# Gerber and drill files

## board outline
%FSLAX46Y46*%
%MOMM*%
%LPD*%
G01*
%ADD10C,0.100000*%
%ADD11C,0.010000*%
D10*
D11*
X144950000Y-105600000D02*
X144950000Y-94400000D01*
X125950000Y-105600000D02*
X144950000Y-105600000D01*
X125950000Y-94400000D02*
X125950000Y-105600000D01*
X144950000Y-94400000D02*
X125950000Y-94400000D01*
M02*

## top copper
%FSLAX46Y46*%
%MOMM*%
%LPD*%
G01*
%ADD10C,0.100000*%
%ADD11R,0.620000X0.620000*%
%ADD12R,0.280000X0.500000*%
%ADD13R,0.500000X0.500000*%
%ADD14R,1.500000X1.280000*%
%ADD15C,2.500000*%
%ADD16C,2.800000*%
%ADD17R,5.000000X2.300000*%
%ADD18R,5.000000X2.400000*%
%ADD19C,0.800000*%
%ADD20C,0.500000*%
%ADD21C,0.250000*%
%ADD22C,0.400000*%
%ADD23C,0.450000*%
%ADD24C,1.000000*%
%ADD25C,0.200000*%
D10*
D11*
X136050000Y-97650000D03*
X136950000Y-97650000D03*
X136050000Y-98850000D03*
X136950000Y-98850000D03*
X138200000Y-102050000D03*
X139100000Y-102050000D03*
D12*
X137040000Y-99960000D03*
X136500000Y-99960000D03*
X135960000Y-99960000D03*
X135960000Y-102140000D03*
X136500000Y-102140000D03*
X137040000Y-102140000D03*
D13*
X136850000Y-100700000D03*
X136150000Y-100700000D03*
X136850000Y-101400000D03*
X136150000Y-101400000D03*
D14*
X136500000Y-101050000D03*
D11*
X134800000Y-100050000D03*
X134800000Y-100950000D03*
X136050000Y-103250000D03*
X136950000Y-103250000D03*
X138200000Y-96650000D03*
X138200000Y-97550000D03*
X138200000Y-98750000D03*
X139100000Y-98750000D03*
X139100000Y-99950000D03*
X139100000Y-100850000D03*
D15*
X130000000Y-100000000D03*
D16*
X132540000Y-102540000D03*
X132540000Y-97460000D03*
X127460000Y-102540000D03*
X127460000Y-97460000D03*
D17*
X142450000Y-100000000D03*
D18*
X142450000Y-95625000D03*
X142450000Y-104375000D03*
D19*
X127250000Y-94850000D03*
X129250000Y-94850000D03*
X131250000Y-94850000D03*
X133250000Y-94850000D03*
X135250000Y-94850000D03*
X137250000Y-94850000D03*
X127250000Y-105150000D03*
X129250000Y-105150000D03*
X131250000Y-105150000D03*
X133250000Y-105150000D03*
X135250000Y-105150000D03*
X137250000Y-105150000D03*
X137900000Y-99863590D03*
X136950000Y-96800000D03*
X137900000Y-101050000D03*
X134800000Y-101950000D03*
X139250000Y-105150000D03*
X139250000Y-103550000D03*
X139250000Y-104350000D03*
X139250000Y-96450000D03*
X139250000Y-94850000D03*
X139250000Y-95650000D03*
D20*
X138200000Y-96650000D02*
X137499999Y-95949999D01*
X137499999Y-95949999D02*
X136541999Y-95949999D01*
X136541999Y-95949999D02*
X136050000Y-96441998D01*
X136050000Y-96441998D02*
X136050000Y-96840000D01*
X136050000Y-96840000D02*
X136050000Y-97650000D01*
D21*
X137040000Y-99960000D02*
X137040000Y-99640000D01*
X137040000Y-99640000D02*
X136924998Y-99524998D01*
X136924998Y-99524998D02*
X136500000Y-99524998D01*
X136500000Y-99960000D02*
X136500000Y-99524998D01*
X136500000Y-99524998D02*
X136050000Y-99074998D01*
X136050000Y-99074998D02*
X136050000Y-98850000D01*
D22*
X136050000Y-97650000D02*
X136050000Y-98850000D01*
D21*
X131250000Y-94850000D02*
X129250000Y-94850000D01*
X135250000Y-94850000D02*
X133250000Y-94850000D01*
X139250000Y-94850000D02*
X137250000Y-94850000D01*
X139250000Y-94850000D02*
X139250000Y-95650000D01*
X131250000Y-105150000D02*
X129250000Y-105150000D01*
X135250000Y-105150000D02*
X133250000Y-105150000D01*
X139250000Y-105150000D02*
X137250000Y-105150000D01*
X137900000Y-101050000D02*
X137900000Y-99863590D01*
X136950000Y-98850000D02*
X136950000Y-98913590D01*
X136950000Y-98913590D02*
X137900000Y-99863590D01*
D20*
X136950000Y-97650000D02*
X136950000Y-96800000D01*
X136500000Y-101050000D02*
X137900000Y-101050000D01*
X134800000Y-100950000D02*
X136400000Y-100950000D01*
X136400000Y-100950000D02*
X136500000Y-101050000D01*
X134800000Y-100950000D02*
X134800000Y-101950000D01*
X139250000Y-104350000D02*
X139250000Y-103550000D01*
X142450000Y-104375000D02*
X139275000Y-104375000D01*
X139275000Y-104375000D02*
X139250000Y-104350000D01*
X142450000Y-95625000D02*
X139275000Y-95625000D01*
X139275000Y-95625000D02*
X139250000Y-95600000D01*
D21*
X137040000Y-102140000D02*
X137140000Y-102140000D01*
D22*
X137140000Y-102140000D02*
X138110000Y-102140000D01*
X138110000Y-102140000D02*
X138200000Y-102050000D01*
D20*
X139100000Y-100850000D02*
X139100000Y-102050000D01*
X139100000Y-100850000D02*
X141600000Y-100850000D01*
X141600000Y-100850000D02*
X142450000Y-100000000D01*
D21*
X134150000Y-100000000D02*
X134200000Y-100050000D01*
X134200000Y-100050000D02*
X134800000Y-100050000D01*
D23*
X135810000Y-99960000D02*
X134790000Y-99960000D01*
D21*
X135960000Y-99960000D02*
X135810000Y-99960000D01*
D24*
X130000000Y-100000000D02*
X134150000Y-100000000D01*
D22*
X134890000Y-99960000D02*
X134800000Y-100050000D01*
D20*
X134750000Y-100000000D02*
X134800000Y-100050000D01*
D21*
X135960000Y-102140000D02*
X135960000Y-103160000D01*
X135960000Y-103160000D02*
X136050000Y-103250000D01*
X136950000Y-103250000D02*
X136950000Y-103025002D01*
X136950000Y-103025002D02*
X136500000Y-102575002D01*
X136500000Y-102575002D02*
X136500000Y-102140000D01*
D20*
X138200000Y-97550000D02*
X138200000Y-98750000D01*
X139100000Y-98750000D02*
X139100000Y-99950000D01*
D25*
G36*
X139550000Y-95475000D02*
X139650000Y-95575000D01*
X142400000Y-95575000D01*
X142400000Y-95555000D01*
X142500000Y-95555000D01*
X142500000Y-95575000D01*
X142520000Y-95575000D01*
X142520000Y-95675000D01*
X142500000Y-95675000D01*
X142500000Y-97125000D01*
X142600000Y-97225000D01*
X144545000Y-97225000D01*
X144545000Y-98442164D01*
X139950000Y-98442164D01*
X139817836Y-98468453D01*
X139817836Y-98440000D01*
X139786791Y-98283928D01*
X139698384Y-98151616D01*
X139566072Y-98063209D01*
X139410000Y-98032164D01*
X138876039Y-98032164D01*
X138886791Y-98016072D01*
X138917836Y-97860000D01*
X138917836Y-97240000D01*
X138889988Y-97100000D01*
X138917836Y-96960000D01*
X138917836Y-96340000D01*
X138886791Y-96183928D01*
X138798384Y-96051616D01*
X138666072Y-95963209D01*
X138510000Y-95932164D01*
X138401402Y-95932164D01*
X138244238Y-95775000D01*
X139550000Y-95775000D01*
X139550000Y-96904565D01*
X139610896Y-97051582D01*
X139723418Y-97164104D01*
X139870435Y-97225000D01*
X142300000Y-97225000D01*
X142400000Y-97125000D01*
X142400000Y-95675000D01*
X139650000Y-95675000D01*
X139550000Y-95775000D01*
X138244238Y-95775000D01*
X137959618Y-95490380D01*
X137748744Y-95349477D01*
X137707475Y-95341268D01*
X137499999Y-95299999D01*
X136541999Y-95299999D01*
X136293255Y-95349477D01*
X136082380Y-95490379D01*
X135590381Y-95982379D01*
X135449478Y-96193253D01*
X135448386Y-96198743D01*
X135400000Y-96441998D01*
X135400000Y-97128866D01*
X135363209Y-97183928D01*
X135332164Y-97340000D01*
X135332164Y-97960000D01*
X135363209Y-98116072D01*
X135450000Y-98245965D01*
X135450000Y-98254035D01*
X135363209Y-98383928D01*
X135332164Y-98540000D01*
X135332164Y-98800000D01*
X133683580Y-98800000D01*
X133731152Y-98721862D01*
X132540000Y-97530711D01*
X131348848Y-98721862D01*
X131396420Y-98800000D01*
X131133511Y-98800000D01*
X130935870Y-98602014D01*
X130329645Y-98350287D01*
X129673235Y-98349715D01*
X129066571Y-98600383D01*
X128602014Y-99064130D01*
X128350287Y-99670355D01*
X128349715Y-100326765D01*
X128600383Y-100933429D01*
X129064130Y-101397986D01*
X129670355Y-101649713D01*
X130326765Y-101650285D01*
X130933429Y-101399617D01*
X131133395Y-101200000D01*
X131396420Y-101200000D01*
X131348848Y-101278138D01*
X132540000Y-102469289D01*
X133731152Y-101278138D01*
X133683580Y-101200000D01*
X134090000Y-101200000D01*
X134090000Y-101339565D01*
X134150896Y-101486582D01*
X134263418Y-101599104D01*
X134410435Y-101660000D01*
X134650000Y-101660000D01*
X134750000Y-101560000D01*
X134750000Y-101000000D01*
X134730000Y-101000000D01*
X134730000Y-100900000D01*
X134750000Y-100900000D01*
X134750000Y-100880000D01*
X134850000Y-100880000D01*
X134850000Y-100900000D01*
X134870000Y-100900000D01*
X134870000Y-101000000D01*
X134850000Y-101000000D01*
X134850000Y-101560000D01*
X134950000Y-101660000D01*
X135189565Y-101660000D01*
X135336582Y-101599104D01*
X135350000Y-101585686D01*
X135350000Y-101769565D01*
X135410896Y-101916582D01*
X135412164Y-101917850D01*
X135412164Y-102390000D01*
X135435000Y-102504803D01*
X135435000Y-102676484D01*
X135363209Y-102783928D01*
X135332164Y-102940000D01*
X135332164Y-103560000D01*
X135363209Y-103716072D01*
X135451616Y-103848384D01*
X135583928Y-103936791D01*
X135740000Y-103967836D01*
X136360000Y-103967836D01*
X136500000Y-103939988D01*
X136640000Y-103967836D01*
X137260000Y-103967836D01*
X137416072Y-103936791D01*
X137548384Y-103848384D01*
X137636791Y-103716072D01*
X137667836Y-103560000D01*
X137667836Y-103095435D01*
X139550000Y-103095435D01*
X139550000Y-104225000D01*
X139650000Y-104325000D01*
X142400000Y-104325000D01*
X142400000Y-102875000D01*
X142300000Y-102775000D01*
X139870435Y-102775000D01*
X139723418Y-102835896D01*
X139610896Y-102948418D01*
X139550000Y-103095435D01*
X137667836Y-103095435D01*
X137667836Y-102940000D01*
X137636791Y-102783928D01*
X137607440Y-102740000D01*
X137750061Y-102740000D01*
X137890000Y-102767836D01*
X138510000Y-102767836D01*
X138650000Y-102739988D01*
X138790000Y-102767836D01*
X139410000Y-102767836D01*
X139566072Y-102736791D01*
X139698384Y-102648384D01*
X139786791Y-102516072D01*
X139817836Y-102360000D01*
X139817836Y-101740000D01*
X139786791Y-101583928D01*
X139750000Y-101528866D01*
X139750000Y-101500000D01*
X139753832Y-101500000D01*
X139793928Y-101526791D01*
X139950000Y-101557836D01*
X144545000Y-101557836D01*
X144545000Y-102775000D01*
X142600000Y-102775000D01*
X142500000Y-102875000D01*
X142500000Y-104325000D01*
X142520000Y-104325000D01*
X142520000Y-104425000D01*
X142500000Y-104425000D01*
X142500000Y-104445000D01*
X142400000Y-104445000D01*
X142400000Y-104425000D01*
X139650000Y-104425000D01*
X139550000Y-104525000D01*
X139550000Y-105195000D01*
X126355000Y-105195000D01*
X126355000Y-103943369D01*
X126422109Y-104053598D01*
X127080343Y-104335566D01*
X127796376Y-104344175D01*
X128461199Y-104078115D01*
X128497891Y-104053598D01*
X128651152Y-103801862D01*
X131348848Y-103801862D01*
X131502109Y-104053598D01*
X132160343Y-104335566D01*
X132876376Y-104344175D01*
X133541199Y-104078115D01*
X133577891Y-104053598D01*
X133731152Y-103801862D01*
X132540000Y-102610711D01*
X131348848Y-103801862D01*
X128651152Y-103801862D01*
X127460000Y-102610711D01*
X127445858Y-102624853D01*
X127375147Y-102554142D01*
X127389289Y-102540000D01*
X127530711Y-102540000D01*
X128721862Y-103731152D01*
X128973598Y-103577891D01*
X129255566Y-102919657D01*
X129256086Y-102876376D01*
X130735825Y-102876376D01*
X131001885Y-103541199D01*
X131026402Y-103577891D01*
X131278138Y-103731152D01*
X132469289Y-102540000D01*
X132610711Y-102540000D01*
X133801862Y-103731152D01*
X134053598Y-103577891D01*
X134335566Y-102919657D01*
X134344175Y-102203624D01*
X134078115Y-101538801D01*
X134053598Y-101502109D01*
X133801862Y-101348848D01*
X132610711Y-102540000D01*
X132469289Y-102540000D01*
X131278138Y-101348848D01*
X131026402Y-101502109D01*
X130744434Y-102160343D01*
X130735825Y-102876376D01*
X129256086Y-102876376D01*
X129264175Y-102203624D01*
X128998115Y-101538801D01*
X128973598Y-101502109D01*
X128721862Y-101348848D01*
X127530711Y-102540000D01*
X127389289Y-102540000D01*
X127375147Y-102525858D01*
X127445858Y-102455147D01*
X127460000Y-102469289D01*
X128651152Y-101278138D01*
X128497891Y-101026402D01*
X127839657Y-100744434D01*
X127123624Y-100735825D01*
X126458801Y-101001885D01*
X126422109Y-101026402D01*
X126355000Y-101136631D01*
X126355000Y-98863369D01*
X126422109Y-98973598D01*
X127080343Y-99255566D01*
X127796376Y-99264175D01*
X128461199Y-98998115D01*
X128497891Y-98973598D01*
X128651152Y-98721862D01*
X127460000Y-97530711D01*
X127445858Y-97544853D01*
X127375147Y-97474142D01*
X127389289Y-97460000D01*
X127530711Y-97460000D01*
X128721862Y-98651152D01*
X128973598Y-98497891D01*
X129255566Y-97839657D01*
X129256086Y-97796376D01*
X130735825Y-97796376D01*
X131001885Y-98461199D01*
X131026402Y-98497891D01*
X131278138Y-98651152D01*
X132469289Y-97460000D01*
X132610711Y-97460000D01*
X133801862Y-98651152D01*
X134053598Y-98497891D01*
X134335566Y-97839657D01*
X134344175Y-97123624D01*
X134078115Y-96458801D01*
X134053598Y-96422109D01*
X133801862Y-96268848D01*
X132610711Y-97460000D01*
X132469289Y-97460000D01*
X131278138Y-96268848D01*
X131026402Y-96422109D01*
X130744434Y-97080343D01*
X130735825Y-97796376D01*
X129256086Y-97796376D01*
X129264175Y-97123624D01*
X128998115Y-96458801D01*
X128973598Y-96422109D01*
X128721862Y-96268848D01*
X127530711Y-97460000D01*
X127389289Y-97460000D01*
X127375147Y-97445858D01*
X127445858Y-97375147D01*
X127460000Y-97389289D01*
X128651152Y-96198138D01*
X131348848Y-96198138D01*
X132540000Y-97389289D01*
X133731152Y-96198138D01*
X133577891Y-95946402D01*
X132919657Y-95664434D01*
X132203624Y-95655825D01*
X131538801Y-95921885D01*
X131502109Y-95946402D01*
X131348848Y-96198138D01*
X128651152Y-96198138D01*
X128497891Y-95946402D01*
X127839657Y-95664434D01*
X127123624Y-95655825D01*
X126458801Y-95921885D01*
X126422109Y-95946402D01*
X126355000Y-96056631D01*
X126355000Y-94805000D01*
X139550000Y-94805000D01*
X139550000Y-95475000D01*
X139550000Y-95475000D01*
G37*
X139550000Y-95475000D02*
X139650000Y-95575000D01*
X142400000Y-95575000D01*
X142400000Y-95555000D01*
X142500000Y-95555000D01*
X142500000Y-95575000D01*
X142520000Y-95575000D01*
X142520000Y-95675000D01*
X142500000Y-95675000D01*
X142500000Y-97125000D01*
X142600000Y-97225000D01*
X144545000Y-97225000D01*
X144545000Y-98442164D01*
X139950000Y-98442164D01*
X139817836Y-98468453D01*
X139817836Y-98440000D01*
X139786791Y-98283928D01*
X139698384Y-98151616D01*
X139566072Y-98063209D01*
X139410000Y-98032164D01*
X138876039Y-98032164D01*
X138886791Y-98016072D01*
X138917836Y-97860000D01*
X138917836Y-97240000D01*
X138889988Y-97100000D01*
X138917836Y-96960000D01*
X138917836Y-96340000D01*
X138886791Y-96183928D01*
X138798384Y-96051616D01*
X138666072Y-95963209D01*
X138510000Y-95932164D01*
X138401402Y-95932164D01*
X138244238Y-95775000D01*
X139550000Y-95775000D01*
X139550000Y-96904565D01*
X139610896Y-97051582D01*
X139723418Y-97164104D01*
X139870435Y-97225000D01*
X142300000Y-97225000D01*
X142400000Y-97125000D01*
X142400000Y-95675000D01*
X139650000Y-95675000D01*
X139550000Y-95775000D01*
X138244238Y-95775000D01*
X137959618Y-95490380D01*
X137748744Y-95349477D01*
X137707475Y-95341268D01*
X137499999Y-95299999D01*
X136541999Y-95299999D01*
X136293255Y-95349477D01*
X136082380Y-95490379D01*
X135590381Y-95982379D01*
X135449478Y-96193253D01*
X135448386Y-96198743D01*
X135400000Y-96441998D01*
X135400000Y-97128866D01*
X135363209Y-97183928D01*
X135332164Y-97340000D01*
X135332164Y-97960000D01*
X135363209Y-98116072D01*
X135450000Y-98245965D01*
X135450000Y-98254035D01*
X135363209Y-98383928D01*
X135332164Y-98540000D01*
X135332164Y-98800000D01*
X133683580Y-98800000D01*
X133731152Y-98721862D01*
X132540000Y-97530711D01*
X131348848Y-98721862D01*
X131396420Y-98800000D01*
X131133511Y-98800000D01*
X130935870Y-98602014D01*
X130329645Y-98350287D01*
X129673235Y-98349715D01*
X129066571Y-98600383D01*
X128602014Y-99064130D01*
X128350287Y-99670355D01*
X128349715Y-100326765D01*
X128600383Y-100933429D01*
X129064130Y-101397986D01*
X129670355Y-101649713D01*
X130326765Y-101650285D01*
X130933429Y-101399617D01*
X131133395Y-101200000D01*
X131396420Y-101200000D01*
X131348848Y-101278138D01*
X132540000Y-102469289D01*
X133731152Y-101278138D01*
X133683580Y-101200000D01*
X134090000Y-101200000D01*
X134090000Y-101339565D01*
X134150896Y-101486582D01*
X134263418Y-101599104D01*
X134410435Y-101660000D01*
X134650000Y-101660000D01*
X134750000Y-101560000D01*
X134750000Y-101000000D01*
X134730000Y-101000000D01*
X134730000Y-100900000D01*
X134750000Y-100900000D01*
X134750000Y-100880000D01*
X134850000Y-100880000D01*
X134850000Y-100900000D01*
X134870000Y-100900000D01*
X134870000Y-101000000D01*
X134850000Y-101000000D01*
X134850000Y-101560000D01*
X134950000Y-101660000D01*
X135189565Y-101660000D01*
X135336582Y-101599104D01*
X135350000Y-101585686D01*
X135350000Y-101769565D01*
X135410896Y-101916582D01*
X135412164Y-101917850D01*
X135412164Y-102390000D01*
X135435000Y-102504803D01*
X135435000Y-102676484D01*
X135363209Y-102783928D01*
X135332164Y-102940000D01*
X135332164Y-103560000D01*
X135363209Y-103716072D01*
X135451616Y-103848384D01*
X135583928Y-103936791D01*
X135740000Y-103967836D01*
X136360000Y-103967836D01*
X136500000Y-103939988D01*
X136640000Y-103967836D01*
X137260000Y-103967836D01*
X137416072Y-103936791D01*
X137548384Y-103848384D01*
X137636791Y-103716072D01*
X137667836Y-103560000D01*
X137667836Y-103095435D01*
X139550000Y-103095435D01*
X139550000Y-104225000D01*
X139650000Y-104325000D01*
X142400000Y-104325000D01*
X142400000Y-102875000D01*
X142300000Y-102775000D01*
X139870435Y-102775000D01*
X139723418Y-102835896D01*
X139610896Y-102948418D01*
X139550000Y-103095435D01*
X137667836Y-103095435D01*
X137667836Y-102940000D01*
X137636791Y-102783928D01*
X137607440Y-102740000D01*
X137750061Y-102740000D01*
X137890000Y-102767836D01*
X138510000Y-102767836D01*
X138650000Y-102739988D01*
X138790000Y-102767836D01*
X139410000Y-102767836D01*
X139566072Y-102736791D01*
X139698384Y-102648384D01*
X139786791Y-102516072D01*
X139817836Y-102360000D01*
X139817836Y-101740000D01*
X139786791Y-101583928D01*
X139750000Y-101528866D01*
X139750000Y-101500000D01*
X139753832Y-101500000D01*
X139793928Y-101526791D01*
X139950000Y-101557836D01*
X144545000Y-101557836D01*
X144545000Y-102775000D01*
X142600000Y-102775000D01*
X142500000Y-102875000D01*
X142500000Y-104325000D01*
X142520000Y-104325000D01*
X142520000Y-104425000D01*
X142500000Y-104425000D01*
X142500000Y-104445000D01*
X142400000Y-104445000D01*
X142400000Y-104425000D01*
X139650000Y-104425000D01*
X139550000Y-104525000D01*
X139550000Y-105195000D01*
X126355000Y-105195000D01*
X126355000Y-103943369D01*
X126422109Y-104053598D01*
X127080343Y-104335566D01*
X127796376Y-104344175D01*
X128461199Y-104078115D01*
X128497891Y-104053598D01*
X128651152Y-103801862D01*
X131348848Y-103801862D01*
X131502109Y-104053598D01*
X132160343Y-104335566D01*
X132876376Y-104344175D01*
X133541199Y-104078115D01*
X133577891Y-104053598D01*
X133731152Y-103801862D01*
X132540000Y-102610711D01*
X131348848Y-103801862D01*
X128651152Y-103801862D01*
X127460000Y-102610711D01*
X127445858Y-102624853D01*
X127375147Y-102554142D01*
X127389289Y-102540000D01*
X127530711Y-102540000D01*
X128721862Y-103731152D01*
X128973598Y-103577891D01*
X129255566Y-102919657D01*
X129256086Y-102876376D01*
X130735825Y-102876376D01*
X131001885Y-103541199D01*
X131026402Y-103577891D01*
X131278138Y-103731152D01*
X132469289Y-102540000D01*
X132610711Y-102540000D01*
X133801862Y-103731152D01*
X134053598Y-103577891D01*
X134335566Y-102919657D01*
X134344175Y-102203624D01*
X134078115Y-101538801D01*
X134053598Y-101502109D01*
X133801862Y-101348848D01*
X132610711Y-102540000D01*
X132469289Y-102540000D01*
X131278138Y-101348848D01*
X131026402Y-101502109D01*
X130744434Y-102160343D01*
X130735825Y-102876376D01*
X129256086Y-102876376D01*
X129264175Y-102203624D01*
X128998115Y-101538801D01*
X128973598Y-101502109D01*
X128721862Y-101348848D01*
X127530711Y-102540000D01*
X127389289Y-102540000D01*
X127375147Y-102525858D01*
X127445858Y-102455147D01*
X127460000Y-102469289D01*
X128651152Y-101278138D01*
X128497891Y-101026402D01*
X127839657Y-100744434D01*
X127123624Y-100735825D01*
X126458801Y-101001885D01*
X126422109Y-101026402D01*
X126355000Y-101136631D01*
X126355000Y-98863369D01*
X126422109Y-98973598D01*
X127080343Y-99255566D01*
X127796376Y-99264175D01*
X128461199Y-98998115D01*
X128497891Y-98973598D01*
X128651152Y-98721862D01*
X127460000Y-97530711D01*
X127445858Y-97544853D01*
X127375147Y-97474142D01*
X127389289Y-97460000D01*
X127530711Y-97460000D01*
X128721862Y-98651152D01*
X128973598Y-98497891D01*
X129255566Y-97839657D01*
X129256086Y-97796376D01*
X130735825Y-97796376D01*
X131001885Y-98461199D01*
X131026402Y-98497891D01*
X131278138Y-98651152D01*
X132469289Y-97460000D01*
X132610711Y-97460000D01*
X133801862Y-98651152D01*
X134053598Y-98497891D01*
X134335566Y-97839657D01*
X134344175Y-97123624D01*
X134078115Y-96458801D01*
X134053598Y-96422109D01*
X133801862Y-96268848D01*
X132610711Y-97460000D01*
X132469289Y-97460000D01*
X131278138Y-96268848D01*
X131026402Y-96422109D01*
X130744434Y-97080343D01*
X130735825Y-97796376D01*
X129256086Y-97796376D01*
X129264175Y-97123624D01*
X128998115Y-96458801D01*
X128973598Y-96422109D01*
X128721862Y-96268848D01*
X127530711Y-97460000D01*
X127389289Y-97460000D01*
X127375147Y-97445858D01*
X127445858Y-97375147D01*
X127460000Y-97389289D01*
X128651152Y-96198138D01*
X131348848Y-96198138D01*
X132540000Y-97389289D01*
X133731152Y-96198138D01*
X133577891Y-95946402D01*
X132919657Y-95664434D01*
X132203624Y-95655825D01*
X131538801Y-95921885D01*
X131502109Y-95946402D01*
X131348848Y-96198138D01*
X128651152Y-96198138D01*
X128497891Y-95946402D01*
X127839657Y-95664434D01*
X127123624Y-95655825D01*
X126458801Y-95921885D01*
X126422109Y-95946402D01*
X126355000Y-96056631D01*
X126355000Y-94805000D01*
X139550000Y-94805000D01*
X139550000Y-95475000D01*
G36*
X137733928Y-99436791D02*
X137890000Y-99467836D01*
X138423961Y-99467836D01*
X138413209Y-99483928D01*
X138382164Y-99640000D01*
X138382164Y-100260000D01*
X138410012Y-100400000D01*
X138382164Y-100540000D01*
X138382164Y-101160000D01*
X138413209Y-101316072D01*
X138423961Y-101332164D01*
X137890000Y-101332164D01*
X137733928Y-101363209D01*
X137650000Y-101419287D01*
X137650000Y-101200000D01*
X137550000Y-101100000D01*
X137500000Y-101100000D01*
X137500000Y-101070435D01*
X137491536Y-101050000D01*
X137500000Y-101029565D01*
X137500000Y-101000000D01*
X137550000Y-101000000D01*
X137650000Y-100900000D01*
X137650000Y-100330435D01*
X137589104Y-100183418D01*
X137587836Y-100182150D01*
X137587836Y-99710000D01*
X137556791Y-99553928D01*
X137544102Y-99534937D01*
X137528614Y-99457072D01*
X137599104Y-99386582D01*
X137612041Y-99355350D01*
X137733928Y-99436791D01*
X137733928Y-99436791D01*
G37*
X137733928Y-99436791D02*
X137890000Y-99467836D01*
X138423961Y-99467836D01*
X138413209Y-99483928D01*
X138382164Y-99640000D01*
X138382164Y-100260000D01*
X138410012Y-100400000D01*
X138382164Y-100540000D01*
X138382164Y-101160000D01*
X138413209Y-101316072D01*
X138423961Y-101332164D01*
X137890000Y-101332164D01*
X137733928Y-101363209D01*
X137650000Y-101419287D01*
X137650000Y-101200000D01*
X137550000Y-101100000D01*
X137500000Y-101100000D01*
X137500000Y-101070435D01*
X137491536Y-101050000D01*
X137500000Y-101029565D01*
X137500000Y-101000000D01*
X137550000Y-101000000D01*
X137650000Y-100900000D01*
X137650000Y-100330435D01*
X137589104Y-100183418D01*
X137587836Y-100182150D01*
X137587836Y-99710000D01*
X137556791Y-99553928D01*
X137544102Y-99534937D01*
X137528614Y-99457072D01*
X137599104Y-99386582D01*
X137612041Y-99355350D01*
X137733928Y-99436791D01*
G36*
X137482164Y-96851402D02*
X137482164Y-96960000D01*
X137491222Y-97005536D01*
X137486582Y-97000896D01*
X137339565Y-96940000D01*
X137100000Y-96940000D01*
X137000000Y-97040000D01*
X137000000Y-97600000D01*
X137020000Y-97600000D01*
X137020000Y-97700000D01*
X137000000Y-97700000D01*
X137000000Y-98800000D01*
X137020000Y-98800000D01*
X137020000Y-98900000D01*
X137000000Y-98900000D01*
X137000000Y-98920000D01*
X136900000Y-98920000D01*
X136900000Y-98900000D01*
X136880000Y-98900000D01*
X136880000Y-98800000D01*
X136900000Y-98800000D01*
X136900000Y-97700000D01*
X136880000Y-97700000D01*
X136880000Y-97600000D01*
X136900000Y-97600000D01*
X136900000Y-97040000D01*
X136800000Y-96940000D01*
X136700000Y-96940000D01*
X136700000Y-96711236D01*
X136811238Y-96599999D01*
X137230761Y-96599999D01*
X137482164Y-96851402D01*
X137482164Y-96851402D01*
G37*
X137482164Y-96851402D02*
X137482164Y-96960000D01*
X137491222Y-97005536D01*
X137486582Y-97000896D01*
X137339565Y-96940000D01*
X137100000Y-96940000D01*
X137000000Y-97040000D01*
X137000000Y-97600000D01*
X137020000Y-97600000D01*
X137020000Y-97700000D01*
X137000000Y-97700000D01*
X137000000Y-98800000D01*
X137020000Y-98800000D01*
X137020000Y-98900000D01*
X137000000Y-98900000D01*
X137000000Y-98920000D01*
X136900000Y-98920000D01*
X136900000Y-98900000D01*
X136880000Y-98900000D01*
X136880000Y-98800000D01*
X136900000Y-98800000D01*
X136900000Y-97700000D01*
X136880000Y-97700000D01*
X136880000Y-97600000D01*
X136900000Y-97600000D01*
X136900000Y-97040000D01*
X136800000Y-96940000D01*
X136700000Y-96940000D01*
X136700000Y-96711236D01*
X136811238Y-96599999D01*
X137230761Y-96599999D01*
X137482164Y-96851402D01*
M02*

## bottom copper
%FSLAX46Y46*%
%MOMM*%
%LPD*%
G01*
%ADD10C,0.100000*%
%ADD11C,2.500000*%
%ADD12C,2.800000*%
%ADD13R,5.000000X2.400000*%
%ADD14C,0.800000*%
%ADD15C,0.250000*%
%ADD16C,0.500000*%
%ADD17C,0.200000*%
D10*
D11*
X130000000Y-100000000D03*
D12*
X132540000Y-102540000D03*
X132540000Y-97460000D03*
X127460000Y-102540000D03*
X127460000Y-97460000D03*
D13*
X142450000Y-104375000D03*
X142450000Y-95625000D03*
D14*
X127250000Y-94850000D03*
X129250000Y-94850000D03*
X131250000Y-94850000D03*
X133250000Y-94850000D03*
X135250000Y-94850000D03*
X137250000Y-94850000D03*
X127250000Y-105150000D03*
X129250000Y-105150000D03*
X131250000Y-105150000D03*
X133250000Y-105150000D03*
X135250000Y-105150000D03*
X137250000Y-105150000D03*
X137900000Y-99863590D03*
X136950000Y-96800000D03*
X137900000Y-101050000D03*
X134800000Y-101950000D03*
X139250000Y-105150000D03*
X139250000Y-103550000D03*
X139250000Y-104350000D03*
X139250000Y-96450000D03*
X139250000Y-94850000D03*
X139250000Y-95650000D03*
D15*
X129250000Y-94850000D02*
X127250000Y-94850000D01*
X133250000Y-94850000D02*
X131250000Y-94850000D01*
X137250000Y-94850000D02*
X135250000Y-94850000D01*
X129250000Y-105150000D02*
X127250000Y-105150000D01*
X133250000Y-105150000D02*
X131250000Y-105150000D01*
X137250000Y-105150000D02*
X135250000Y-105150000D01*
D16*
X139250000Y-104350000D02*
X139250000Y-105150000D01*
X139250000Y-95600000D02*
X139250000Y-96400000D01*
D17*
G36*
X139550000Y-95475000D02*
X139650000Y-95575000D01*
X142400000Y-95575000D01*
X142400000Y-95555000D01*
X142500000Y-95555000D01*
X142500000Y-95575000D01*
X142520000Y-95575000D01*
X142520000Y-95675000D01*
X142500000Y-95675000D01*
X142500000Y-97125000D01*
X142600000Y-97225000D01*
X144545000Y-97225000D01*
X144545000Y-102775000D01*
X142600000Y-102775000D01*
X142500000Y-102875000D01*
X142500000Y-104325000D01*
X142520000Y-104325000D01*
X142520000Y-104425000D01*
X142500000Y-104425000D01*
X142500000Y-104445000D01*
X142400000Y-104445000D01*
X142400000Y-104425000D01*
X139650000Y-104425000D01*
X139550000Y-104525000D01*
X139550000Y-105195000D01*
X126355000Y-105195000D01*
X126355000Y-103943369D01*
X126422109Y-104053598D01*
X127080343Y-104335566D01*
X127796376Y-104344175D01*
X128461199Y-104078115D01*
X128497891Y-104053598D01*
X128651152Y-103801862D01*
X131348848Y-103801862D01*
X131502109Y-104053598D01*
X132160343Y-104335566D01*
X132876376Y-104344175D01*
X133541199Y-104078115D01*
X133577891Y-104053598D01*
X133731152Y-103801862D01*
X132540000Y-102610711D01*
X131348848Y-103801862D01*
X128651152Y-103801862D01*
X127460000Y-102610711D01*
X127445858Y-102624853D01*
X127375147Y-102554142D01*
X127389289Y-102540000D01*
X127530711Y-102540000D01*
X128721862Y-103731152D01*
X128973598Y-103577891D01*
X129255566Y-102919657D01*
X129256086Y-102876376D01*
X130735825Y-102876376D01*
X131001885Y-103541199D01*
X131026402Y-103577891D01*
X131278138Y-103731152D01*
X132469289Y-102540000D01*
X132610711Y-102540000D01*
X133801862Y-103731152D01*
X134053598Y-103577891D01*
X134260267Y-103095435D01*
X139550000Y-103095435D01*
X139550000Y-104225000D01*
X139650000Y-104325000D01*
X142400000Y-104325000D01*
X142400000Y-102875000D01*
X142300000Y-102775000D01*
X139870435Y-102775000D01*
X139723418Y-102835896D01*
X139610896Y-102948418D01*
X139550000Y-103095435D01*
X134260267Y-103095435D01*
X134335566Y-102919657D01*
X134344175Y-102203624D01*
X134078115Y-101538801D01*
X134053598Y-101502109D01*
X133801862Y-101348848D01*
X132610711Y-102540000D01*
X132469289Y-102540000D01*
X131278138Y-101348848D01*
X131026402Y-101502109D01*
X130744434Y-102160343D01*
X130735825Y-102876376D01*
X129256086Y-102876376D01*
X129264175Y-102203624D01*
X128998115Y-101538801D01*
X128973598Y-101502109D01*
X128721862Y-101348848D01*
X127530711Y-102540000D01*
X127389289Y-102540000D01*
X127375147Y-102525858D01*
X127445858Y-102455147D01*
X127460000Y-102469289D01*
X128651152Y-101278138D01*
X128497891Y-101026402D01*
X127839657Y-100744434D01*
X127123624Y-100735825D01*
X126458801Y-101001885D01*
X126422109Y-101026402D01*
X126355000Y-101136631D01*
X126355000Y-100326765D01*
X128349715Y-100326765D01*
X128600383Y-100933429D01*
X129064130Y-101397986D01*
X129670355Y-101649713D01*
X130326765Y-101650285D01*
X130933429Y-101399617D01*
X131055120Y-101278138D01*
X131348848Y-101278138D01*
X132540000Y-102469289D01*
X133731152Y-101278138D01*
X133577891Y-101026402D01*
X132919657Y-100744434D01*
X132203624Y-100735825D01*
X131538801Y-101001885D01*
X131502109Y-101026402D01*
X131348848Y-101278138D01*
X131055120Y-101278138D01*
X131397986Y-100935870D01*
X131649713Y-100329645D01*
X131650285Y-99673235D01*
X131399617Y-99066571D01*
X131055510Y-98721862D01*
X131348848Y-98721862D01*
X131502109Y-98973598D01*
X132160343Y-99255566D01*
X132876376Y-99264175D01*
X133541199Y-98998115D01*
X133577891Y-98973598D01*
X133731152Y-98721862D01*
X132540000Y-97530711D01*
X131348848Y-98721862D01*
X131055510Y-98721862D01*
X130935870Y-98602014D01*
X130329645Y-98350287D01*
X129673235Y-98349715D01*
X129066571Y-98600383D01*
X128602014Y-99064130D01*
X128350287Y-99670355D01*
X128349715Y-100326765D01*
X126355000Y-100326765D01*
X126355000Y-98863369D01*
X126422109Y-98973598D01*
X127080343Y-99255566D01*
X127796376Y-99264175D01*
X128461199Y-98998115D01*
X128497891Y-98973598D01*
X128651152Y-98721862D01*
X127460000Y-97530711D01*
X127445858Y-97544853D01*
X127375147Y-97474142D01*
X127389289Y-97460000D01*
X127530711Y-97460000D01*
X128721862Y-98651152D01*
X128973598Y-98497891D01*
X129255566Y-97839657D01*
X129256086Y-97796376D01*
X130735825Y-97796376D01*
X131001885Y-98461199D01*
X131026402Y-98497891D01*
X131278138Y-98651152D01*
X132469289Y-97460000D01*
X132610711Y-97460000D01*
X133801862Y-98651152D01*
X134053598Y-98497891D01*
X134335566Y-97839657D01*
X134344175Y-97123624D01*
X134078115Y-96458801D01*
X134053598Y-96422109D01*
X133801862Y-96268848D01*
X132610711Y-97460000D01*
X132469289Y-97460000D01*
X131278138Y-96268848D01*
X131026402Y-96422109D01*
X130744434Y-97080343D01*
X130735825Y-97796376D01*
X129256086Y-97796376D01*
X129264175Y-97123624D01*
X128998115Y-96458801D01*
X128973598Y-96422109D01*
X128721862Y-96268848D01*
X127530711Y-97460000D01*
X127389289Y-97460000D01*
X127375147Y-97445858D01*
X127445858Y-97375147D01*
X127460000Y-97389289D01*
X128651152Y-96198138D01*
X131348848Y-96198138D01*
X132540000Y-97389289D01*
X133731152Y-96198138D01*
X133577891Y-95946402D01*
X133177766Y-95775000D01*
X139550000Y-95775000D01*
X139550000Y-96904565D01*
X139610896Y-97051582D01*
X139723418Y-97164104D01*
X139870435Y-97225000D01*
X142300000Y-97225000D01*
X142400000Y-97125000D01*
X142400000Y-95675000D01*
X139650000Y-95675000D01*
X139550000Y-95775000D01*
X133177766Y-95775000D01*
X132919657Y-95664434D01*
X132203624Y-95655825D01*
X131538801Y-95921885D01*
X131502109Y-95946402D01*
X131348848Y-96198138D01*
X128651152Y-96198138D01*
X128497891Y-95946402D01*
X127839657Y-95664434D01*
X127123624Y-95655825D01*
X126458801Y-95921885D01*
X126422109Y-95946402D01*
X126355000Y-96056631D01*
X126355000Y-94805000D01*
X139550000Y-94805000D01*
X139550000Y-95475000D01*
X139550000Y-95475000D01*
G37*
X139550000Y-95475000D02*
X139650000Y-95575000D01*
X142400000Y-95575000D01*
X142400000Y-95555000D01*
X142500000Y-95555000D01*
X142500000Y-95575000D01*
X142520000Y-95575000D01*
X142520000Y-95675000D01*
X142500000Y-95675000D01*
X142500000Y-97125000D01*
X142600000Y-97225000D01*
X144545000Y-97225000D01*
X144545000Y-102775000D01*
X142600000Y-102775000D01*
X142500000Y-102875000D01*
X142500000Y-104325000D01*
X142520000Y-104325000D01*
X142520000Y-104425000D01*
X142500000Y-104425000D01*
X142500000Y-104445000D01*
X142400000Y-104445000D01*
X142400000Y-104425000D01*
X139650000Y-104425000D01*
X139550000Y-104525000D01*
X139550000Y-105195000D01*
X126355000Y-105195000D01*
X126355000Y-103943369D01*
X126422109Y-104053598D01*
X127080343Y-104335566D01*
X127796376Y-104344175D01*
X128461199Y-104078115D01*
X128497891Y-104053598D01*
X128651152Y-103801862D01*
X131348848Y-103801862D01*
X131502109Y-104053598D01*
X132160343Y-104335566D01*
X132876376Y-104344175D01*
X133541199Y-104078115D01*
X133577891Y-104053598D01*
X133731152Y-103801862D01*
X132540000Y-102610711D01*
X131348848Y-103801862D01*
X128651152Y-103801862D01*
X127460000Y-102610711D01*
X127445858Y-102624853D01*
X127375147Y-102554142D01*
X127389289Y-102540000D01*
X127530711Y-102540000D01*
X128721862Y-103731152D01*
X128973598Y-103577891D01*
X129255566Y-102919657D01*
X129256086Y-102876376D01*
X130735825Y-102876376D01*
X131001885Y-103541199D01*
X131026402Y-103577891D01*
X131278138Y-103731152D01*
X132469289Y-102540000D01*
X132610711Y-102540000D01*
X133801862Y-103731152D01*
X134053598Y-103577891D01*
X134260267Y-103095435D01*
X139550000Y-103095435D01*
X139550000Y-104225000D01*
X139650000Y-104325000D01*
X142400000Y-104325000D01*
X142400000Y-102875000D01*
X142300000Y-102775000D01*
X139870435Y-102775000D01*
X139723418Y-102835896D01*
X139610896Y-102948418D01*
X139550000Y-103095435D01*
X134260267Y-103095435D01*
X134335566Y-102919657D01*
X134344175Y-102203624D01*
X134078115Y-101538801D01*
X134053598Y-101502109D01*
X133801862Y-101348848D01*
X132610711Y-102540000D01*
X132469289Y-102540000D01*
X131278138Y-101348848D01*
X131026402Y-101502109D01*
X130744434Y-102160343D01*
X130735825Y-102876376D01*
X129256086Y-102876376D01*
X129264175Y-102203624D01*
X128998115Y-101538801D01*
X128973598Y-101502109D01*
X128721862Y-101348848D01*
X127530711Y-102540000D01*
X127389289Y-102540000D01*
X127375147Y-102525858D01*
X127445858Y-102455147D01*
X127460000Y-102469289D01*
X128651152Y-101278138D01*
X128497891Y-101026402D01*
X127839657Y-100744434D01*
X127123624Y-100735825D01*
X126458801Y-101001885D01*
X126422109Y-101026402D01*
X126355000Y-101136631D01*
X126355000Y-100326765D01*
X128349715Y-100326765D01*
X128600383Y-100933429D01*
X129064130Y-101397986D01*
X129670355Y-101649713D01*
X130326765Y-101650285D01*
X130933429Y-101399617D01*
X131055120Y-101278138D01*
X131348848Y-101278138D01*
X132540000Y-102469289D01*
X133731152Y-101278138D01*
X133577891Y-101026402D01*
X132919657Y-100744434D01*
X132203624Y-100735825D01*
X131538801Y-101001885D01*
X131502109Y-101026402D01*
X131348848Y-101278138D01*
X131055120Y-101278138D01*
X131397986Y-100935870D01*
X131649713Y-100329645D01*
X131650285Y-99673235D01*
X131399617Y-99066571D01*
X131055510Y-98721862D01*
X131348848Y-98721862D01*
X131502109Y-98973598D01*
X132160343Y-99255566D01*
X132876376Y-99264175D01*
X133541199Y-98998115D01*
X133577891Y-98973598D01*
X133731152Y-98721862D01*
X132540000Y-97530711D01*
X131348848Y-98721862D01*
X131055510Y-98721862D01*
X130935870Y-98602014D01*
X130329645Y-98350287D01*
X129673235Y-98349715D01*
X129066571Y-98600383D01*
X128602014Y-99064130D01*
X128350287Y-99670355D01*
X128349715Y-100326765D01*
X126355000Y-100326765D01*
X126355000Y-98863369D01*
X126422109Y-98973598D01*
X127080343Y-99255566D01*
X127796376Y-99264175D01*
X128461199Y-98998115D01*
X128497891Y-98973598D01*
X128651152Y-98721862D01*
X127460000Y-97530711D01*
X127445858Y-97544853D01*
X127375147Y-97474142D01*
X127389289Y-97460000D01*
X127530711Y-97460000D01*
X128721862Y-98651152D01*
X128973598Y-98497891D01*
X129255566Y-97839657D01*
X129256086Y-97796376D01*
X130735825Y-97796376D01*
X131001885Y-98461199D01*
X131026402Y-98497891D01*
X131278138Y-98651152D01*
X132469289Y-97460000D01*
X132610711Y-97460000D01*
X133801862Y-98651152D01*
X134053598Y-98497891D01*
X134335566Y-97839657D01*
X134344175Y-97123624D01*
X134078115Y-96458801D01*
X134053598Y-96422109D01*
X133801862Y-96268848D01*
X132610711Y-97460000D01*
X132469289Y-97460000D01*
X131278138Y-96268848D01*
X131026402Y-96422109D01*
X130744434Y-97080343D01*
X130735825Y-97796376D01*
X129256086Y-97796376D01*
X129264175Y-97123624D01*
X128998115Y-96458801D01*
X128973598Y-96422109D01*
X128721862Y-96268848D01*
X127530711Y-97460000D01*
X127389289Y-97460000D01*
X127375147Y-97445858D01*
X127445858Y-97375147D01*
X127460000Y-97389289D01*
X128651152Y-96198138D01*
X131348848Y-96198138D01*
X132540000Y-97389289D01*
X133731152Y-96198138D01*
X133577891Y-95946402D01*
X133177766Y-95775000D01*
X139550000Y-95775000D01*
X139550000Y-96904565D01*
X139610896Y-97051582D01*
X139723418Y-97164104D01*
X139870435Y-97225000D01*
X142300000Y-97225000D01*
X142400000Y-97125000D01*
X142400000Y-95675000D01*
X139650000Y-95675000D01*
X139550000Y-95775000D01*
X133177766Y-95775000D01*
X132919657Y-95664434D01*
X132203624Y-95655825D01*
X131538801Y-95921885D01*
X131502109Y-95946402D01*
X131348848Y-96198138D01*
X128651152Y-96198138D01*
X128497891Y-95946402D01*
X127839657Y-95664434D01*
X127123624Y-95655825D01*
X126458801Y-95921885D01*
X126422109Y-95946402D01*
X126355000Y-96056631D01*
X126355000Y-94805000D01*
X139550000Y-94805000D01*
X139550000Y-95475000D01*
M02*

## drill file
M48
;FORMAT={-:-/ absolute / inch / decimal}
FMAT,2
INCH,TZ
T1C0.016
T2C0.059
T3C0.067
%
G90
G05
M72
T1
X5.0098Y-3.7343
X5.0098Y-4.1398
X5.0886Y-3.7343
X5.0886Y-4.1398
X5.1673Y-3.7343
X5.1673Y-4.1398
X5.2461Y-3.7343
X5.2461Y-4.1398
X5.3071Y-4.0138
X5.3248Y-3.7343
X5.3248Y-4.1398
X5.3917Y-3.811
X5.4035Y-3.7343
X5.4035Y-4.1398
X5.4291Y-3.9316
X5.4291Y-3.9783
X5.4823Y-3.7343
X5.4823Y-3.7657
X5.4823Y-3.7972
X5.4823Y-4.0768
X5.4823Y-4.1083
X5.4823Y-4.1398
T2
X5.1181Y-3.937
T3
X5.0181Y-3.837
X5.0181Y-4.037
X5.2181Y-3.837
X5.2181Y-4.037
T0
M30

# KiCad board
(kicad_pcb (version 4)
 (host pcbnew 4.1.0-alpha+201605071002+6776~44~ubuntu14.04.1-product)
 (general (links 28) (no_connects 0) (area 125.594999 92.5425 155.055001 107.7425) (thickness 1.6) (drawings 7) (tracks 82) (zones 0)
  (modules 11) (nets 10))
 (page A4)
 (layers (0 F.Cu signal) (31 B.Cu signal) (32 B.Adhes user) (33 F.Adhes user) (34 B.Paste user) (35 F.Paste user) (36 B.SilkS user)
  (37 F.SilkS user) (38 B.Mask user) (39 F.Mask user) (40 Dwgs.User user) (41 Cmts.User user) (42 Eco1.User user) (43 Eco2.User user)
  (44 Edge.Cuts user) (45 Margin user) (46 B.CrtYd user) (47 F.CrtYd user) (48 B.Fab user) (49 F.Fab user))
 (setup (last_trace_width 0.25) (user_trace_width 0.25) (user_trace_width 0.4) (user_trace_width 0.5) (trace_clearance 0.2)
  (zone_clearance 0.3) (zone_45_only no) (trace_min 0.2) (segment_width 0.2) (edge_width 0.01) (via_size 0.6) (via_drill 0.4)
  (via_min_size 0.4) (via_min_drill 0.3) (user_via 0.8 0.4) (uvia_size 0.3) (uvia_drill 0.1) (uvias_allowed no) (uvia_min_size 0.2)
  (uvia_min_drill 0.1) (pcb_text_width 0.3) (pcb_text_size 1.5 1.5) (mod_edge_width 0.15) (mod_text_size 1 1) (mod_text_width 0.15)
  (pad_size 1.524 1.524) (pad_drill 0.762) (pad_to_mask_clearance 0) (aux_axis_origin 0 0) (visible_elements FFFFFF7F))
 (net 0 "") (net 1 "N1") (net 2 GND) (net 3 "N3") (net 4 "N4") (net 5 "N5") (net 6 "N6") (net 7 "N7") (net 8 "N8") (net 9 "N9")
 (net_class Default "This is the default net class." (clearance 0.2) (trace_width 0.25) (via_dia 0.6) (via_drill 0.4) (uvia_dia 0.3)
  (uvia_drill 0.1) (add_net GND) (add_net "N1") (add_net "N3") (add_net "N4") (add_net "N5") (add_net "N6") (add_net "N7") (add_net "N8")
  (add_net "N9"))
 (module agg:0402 (layer F.Cu) (at 136.5 97.65)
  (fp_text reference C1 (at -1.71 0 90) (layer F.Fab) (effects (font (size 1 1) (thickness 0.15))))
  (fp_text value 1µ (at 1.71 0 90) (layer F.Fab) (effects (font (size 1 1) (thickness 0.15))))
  (pad 1 smd rect (at -0.45 0) (size 0.62 0.62) (layers F.Cu F.Paste F.Mask) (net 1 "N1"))
  (pad 2 smd rect (at 0.45 0) (size 0.62 0.62) (layers F.Cu F.Paste F.Mask) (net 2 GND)))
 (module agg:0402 (layer F.Cu) (at 136.5 98.85)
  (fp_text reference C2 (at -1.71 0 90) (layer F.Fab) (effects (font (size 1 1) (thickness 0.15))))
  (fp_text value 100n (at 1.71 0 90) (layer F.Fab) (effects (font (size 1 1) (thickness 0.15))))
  (pad 1 smd rect (at -0.45 0) (size 0.62 0.62) (layers F.Cu F.Paste F.Mask) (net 1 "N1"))
  (pad 2 smd rect (at 0.45 0) (size 0.62 0.62) (layers F.Cu F.Paste F.Mask) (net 2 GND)))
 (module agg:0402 (layer F.Cu) (at 138.65 102.05)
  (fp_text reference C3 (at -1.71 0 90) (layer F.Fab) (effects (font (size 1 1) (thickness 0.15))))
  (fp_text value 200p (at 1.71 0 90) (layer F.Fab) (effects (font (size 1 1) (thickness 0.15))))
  (pad 1 smd rect (at -0.45 0) (size 0.62 0.62) (layers F.Cu F.Paste F.Mask) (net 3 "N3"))
  (pad 2 smd rect (at 0.45 0) (size 0.62 0.62) (layers F.Cu F.Paste F.Mask) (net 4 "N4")))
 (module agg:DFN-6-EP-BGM (layer F.Cu) (at 136.5 101.05 270)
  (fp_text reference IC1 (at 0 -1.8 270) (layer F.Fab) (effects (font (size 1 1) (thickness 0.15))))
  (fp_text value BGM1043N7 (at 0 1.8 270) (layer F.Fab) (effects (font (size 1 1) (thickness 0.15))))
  (pad 1 smd rect (at -1.09 -0.54 270) (size 0.5 0.28) (layers F.Cu F.Paste F.Mask) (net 1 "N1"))
  (pad 2 smd rect (at -1.09 0 270) (size 0.5 0.28) (layers F.Cu F.Paste F.Mask) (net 1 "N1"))
  (pad 3 smd rect (at -1.09 0.54 270) (size 0.5 0.28) (layers F.Cu F.Paste F.Mask) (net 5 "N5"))
  (pad 4 smd rect (at 1.09 0.54 270) (size 0.5 0.28) (layers F.Cu F.Paste F.Mask) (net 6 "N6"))
  (pad 5 smd rect (at 1.09 0 270) (size 0.5 0.28) (layers F.Cu F.Paste F.Mask) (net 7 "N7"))
  (pad 6 smd rect (at 1.09 -0.54 270) (size 0.5 0.28) (layers F.Cu F.Paste F.Mask) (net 3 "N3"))
  (pad EP smd rect (at -0.35 -0.35 270) (size 0.5 0.5) (layers F.Cu F.Paste) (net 2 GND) (solder_paste_margin 0.001))
  (pad EP smd rect (at -0.35 0.35 270) (size 0.5 0.5) (layers F.Cu F.Paste) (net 2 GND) (solder_paste_margin 0.001))
  (pad EP smd rect (at 0.35 -0.35 270) (size 0.5 0.5) (layers F.Cu F.Paste) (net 2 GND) (solder_paste_margin 0.001))
  (pad EP smd rect (at 0.35 0.35 270) (size 0.5 0.5) (layers F.Cu F.Paste) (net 2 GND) (solder_paste_margin 0.001))
  (pad EP smd rect (at 0 0 270) (size 1.28 1.5) (layers F.Cu F.Mask) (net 2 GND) (solder_mask_margin 0.001)))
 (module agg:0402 (layer F.Cu) (at 134.8 100.5 270)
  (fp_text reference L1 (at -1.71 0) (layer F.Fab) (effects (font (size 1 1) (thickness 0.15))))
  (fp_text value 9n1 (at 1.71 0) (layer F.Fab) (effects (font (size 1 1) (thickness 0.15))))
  (pad 1 smd rect (at -0.45 0 270) (size 0.62 0.62) (layers F.Cu F.Paste F.Mask) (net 5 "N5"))
  (pad 2 smd rect (at 0.45 0 270) (size 0.62 0.62) (layers F.Cu F.Paste F.Mask) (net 2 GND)))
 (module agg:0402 (layer F.Cu) (at 136.5 103.25)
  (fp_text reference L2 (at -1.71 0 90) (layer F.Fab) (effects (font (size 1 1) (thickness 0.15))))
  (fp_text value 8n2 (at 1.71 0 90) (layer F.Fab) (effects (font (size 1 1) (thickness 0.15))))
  (pad 1 smd rect (at -0.45 0) (size 0.62 0.62) (layers F.Cu F.Paste F.Mask) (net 6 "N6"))
  (pad 2 smd rect (at 0.45 0) (size 0.62 0.62) (layers F.Cu F.Paste F.Mask) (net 7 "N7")))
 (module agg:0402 (layer F.Cu) (at 138.2 97.1 270)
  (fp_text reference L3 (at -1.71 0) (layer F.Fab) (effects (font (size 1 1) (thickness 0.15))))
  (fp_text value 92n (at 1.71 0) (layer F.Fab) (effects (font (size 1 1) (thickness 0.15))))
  (pad 1 smd rect (at -0.45 0 270) (size 0.62 0.62) (layers F.Cu F.Paste F.Mask) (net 1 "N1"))
  (pad 2 smd rect (at 0.45 0 270) (size 0.62 0.62) (layers F.Cu F.Paste F.Mask) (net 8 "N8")))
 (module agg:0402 (layer F.Cu) (at 138.65 98.75)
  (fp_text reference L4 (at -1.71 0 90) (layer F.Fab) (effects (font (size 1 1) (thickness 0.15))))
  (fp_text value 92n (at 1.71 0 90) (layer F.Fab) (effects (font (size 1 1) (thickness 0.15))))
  (pad 1 smd rect (at -0.45 0) (size 0.62 0.62) (layers F.Cu F.Paste F.Mask) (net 8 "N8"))
  (pad 2 smd rect (at 0.45 0) (size 0.62 0.62) (layers F.Cu F.Paste F.Mask) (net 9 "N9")))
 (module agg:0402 (layer F.Cu) (at 139.1 100.4 270)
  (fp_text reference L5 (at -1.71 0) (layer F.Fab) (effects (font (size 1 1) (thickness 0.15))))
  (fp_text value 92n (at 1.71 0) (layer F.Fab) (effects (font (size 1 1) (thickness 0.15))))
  (pad 1 smd rect (at -0.45 0 270) (size 0.62 0.62) (layers F.Cu F.Paste F.Mask) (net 9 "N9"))
  (pad 2 smd rect (at 0.45 0 270) (size 0.62 0.62) (layers F.Cu F.Paste F.Mask) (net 4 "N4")))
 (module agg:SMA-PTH (layer F.Cu) (at 130 100)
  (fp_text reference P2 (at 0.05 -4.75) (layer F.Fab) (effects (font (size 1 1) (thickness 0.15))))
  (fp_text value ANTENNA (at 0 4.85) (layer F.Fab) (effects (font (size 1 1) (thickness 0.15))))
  (pad 1 thru_hole circle (at 0 0) (size 2.5 2.5) (drill 1.5) (layers *.Cu *.Mask F.SilkS) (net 5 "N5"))
  (pad 2 thru_hole circle (at 2.54 2.54) (size 2.8 2.8) (drill 1.7) (layers *.Cu *.Mask F.SilkS) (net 2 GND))
  (pad 2 thru_hole circle (at 2.54 -2.54) (size 2.8 2.8) (drill 1.7) (layers *.Cu *.Mask F.SilkS) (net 2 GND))
  (pad 2 thru_hole circle (at -2.54 2.54) (size 2.8 2.8) (drill 1.7) (layers *.Cu *.Mask F.SilkS) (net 2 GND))
  (pad 2 thru_hole circle (at -2.54 -2.54) (size 2.8 2.8) (drill 1.7) (layers *.Cu *.Mask F.SilkS) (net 2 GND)))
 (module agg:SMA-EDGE (layer F.Cu) (at 142.45 100 270)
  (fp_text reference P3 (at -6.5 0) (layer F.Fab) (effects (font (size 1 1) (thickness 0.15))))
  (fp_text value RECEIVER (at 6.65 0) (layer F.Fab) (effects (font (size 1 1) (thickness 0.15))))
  (pad 1 smd rect (at 0 0 270) (size 2.3 5) (layers F.Cu F.Paste F.Mask) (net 4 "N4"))
  (pad 2 smd rect (at 4.375 0 270) (size 2.4 5) (layers B.Cu B.Paste B.Mask) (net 2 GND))
  (pad 2 smd rect (at -4.375 0 270) (size 2.4 5) (layers B.Cu B.Paste B.Mask) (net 2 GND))
  (pad 2 smd rect (at -4.375 0 270) (size 2.4 5) (layers F.Cu F.Paste F.Mask) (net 2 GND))
  (pad 2 smd rect (at 4.375 0 270) (size 2.4 5) (layers F.Cu F.Paste F.Mask) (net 2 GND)))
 (gr_line (start 144.95 105.6) (end 144.95 94.4) (layer Edge.Cuts) (width 0.01))
 (gr_line (start 125.95 105.6) (end 144.95 105.6) (layer Edge.Cuts) (width 0.01))
 (gr_line (start 125.95 94.4) (end 125.95 105.6) (layer Edge.Cuts) (width 0.01))
 (gr_line (start 144.95 94.4) (end 125.95 94.4) (layer Edge.Cuts) (width 0.01))
 (segment (start 138.2 96.65) (end 137.499999 95.949999) (width 0.5) (layer F.Cu) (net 1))
 (segment (start 137.499999 95.949999) (end 136.541999 95.949999) (width 0.5) (layer F.Cu) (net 1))
 (segment (start 136.541999 95.949999) (end 136.05 96.441998) (width 0.5) (layer F.Cu) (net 1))
 (segment (start 136.05 96.441998) (end 136.05 96.84) (width 0.5) (layer F.Cu) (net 1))
 (segment (start 136.05 96.84) (end 136.05 97.65) (width 0.5) (layer F.Cu) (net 1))
 (segment (start 137.04 99.96) (end 137.04 99.64) (width 0.25) (layer F.Cu) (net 1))
 (segment (start 137.04 99.64) (end 136.924998 99.524998) (width 0.25) (layer F.Cu) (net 1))
 (segment (start 136.924998 99.524998) (end 136.5 99.524998) (width 0.25) (layer F.Cu) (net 1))
 (segment (start 136.5 99.96) (end 136.5 99.524998) (width 0.25) (layer F.Cu) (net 1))
 (segment (start 136.5 99.524998) (end 136.05 99.074998) (width 0.25) (layer F.Cu) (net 1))
 (segment (start 136.05 99.074998) (end 136.05 98.85) (width 0.25) (layer F.Cu) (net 1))
 (segment (start 136.05 97.65) (end 136.05 98.85) (width 0.4) (layer F.Cu) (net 1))
 (segment (start 129.25 94.85) (end 127.25 94.85) (width 0.25) (layer B.Cu) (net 2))
 (via (at 127.25 94.85) (size 0.8) (drill 0.4) (layers F.Cu B.Cu) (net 2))
 (segment (start 131.25 94.85) (end 129.25 94.85) (width 0.25) (layer F.Cu) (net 2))
 (via (at 129.25 94.85) (size 0.8) (drill 0.4) (layers F.Cu B.Cu) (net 2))
 (segment (start 133.25 94.85) (end 131.25 94.85) (width 0.25) (layer B.Cu) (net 2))
 (via (at 131.25 94.85) (size 0.8) (drill 0.4) (layers F.Cu B.Cu) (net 2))
 (segment (start 135.25 94.85) (end 133.25 94.85) (width 0.25) (layer F.Cu) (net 2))
 (via (at 133.25 94.85) (size 0.8) (drill 0.4) (layers F.Cu B.Cu) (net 2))
 (segment (start 137.25 94.85) (end 135.25 94.85) (width 0.25) (layer B.Cu) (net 2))
 (via (at 135.25 94.85) (size 0.8) (drill 0.4) (layers F.Cu B.Cu) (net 2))
 (segment (start 139.25 94.85) (end 137.25 94.85) (width 0.25) (layer F.Cu) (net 2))
 (via (at 137.25 94.85) (size 0.8) (drill 0.4) (layers F.Cu B.Cu) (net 2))
 (segment (start 139.25 94.85) (end 139.25 95.65) (width 0.25) (layer F.Cu) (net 2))
 (segment (start 129.25 105.15) (end 127.25 105.15) (width 0.25) (layer B.Cu) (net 2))
 (via (at 127.25 105.15) (size 0.8) (drill 0.4) (layers F.Cu B.Cu) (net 2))
 (segment (start 131.25 105.15) (end 129.25 105.15) (width 0.25) (layer F.Cu) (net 2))
 (via (at 129.25 105.15) (size 0.8) (drill 0.4) (layers F.Cu B.Cu) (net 2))
 (segment (start 133.25 105.15) (end 131.25 105.15) (width 0.25) (layer B.Cu) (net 2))
 (via (at 131.25 105.15) (size 0.8) (drill 0.4) (layers F.Cu B.Cu) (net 2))
 (segment (start 135.25 105.15) (end 133.25 105.15) (width 0.25) (layer F.Cu) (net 2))
 (via (at 133.25 105.15) (size 0.8) (drill 0.4) (layers F.Cu B.Cu) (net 2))
 (segment (start 137.25 105.15) (end 135.25 105.15) (width 0.25) (layer B.Cu) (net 2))
 (via (at 135.25 105.15) (size 0.8) (drill 0.4) (layers F.Cu B.Cu) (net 2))
 (segment (start 139.25 105.15) (end 137.25 105.15) (width 0.25) (layer F.Cu) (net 2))
 (via (at 137.25 105.15) (size 0.8) (drill 0.4) (layers F.Cu B.Cu) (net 2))
 (segment (start 137.9 101.05) (end 137.9 99.86359) (width 0.25) (layer F.Cu) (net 2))
 (via (at 137.9 99.86359) (size 0.8) (drill 0.4) (layers F.Cu B.Cu) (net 2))
 (segment (start 136.95 98.85) (end 136.95 98.91359) (width 0.25) (layer F.Cu) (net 2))
 (segment (start 136.95 98.91359) (end 137.9 99.86359) (width 0.25) (layer F.Cu) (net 2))
 (segment (start 136.95 97.65) (end 136.95 96.8) (width 0.5) (layer F.Cu) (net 2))
 (via (at 136.95 96.8) (size 0.8) (drill 0.4) (layers F.Cu B.Cu) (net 2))
 (segment (start 136.5 101.05) (end 137.9 101.05) (width 0.5) (layer F.Cu) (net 2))
 (via (at 137.9 101.05) (size 0.8) (drill 0.4) (layers F.Cu B.Cu) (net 2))
 (segment (start 134.8 100.95) (end 136.4 100.95) (width 0.5) (layer F.Cu) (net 2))
 (segment (start 136.4 100.95) (end 136.5 101.05) (width 0.5) (layer F.Cu) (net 2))
 (segment (start 134.8 100.95) (end 134.8 101.95) (width 0.5) (layer F.Cu) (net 2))
 (via (at 134.8 101.95) (size 0.8) (drill 0.4) (layers F.Cu B.Cu) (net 2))
 (segment (start 139.25 104.35) (end 139.25 105.15) (width 0.5) (layer B.Cu) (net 2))
 (via (at 139.25 105.15) (size 0.8) (drill 0.4) (layers F.Cu B.Cu) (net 2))
 (segment (start 139.25 104.35) (end 139.25 103.55) (width 0.5) (layer F.Cu) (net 2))
 (via (at 139.25 103.55) (size 0.8) (drill 0.4) (layers F.Cu B.Cu) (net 2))
 (segment (start 142.45 104.375) (end 139.275 104.375) (width 0.5) (layer F.Cu) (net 2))
 (segment (start 139.275 104.375) (end 139.25 104.35) (width 0.5) (layer F.Cu) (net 2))
 (via (at 139.25 104.35) (size 0.8) (drill 0.4) (layers F.Cu B.Cu) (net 2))
 (segment (start 139.25 95.6) (end 139.25 96.4) (width 0.5) (layer B.Cu) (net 2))
 (via (at 139.25 96.45) (size 0.8) (drill 0.4) (layers F.Cu B.Cu) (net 2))
 (via (at 139.25 94.85) (size 0.8) (drill 0.4) (layers F.Cu B.Cu) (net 2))
 (segment (start 142.45 95.625) (end 139.275 95.625) (width 0.5) (layer F.Cu) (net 2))
 (segment (start 139.275 95.625) (end 139.25 95.6) (width 0.5) (layer F.Cu) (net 2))
 (via (at 139.25 95.65) (size 0.8) (drill 0.4) (layers F.Cu B.Cu) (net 2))
 (segment (start 137.04 102.14) (end 137.14 102.14) (width 0.25) (layer F.Cu) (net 3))
 (segment (start 137.14 102.14) (end 138.11 102.14) (width 0.4) (layer F.Cu) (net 3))
 (segment (start 138.11 102.14) (end 138.2 102.05) (width 0.4) (layer F.Cu) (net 3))
 (segment (start 139.1 100.85) (end 139.1 102.05) (width 0.5) (layer F.Cu) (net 4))
 (segment (start 139.1 100.85) (end 141.6 100.85) (width 0.5) (layer F.Cu) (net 4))
 (segment (start 141.6 100.85) (end 142.45 100) (width 0.5) (layer F.Cu) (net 4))
 (segment (start 134.15 100) (end 134.2 100.05) (width 0.25) (layer F.Cu) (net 5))
 (segment (start 134.2 100.05) (end 134.8 100.05) (width 0.25) (layer F.Cu) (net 5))
 (segment (start 135.81 99.96) (end 134.79 99.96) (width 0.45) (layer F.Cu) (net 5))
 (segment (start 135.96 99.96) (end 135.81 99.96) (width 0.25) (layer F.Cu) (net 5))
 (segment (start 130 100) (end 134.15 100) (width 1) (layer F.Cu) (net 5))
 (segment (start 134.89 99.96) (end 134.8 100.05) (width 0.4) (layer F.Cu) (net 5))
 (segment (start 134.75 100) (end 134.8 100.05) (width 0.5) (layer F.Cu) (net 5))
 (segment (start 135.96 102.14) (end 135.96 103.16) (width 0.25) (layer F.Cu) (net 6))
 (segment (start 135.96 103.16) (end 136.05 103.25) (width 0.25) (layer F.Cu) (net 6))
 (segment (start 136.95 103.25) (end 136.95 103.025002) (width 0.25) (layer F.Cu) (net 7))
 (segment (start 136.95 103.025002) (end 136.5 102.575002) (width 0.25) (layer F.Cu) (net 7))
 (segment (start 136.5 102.575002) (end 136.5 102.14) (width 0.25) (layer F.Cu) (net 7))
 (segment (start 138.2 97.55) (end 138.2 98.75) (width 0.5) (layer F.Cu) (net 8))
 (segment (start 139.1 98.75) (end 139.1 99.95) (width 0.5) (layer F.Cu) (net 9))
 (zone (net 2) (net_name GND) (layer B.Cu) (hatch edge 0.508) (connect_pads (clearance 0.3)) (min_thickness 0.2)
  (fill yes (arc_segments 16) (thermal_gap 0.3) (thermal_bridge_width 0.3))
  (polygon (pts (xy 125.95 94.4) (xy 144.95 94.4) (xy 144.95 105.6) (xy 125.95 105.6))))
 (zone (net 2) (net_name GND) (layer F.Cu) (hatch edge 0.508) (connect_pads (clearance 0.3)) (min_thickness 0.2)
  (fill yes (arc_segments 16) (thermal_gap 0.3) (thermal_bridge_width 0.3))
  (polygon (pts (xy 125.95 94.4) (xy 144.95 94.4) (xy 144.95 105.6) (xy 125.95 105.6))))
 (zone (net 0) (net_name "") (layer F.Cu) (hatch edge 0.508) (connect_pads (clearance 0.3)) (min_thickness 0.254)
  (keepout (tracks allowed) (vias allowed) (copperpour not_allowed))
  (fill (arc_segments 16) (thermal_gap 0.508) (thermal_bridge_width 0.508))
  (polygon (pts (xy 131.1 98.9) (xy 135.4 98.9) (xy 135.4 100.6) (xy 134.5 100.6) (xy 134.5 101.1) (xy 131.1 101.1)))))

